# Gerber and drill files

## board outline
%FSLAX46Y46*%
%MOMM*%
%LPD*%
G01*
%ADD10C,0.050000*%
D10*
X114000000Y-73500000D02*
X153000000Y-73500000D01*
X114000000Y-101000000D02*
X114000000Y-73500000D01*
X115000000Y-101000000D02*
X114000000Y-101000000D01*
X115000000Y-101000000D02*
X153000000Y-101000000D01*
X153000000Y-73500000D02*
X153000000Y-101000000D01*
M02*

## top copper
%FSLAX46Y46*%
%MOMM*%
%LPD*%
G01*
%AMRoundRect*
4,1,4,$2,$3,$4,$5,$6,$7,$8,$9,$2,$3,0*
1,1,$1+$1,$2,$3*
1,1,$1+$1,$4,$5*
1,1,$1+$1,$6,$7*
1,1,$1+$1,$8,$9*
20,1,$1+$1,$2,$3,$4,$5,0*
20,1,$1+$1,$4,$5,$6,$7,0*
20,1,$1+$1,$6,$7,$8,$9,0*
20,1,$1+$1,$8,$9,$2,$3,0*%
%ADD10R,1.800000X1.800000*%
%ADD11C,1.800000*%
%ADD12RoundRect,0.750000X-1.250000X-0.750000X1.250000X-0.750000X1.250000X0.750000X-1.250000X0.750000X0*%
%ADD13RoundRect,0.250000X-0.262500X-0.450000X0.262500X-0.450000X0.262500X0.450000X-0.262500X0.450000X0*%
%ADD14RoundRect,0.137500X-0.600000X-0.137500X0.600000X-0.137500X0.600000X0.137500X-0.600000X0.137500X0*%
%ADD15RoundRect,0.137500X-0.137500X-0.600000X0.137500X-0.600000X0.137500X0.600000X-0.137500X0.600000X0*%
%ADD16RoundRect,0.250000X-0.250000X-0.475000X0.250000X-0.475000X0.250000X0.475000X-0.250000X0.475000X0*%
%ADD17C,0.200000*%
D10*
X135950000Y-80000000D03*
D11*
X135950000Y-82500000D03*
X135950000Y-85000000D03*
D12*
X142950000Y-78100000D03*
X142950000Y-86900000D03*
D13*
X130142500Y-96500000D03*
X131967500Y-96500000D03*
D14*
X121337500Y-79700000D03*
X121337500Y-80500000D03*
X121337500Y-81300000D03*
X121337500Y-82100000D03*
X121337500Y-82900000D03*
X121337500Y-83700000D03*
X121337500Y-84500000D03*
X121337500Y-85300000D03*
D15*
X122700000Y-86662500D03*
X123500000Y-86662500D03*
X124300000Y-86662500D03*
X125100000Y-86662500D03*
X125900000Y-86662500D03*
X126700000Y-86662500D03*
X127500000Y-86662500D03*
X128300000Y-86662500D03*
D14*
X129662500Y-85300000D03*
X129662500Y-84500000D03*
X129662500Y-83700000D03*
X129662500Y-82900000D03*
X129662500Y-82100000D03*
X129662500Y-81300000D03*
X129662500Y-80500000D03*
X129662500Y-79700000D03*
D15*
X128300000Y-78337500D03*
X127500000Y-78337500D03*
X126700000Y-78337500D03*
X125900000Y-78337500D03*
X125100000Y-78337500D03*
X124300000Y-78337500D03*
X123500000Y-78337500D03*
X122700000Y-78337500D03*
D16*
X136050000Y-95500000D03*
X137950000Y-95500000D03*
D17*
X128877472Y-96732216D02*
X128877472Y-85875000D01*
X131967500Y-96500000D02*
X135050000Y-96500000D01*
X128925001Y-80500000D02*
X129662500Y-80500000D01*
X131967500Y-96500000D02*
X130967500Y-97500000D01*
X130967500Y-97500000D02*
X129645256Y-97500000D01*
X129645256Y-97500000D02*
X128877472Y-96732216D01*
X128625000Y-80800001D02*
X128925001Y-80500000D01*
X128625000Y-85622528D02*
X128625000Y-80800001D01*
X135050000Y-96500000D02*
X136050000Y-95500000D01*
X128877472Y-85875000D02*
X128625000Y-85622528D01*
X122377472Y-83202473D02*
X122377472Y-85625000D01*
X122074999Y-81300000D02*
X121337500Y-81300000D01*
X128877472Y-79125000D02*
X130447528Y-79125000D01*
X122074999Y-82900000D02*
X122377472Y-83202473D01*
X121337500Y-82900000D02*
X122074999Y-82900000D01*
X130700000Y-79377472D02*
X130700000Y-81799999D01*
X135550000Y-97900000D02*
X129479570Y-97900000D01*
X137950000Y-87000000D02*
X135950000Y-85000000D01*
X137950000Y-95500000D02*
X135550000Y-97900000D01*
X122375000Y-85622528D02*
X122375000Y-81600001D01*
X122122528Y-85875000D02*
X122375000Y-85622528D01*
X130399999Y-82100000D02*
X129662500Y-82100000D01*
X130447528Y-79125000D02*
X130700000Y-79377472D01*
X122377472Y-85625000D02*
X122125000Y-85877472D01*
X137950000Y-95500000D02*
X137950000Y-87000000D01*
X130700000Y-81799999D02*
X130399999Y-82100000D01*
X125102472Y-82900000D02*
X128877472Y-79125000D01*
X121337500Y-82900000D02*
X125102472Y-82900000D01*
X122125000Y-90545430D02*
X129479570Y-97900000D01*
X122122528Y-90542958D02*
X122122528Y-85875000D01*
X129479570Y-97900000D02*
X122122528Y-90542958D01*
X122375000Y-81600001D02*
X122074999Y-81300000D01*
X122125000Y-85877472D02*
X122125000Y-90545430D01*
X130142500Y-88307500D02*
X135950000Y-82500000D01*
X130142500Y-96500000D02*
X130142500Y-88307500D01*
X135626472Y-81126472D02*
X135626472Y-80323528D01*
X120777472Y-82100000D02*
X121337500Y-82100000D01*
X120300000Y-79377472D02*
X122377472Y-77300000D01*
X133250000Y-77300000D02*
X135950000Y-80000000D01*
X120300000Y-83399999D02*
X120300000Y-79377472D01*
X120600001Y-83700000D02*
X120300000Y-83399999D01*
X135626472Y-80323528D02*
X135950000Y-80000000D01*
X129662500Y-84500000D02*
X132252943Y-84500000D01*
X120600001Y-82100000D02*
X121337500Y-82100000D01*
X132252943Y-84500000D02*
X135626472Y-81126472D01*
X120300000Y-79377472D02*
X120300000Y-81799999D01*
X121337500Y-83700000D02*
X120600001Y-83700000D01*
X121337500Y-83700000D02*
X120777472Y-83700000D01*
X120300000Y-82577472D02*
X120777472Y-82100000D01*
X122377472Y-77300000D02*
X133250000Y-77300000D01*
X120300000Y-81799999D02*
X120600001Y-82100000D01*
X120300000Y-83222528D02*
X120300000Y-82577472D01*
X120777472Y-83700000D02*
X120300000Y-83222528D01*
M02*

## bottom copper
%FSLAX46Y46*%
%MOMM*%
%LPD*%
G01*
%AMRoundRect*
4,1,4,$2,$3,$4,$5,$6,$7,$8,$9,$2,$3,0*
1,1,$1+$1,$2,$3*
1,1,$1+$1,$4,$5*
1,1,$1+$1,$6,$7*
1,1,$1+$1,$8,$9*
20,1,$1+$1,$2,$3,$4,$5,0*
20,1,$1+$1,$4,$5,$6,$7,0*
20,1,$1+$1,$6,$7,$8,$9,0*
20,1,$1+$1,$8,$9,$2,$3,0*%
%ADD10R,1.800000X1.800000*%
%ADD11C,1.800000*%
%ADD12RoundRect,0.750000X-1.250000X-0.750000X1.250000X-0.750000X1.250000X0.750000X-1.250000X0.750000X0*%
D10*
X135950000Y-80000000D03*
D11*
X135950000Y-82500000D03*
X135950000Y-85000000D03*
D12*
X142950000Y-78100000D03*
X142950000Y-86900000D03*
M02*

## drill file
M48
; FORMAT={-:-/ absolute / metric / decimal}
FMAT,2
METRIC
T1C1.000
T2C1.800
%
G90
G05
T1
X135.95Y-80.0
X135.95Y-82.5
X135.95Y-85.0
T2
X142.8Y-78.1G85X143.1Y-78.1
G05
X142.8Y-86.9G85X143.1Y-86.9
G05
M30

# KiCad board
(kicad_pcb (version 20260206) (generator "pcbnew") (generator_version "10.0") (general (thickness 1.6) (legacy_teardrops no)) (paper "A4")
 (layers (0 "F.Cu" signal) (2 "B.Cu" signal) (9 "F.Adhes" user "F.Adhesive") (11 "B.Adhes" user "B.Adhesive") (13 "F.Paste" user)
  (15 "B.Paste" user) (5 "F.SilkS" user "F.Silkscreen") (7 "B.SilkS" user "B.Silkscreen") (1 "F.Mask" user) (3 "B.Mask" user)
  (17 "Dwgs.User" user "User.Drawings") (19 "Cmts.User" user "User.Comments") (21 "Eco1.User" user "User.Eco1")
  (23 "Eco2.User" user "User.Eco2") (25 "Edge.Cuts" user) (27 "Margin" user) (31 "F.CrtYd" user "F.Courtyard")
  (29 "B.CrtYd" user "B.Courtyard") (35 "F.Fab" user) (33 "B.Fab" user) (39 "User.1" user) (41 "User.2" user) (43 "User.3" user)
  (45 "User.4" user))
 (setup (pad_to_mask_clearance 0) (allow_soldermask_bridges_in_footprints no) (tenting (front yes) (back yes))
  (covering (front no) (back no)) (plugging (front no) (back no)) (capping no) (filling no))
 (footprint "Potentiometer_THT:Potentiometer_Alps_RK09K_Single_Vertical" (layer "F.Cu") (at 135.95 80)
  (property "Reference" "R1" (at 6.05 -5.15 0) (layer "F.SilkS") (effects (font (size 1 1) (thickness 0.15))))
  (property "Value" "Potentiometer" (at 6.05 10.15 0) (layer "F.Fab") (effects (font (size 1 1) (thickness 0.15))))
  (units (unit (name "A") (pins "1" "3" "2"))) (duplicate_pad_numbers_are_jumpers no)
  (pad "1" thru_hole rect (at 0 0) (size 1.8 1.8) (drill 1) (layers "*.Cu" "*.Mask") (remove_unused_layers no) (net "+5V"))
  (pad "2" thru_hole circle (at 0 2.5) (size 1.8 1.8) (drill 1) (layers "*.Cu" "*.Mask") (remove_unused_layers no) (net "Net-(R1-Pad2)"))
  (pad "3" thru_hole circle (at 0 5) (size 1.8 1.8) (drill 1) (layers "*.Cu" "*.Mask") (remove_unused_layers no) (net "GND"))
  (pad "MP" thru_hole roundrect (at 7 -1.9) (size 4 3) (drill oval 2.1 1.8) (layers "*.Cu" "*.Mask") (remove_unused_layers no)
   (roundrect_rratio 0.25))
  (pad "MP" thru_hole roundrect (at 7 6.9) (size 4 3) (drill oval 2.1 1.8) (layers "*.Cu" "*.Mask") (remove_unused_layers no)
   (roundrect_rratio 0.25)))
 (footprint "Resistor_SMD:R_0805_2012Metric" (layer "F.Cu") (at 131.055 96.5)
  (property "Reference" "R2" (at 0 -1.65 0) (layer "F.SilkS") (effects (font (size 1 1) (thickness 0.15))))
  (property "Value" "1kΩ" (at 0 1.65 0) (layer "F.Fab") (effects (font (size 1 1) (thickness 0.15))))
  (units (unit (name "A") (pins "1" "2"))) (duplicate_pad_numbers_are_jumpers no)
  (pad "1" smd roundrect (at -0.9125 0) (size 1.025 1.4) (layers "F.Cu" "F.Mask" "F.Paste") (roundrect_rratio 0.243902)
   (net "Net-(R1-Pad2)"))
  (pad "2" smd roundrect (at 0.9125 0) (size 1.025 1.4) (layers "F.Cu" "F.Mask" "F.Paste") (roundrect_rratio 0.243902) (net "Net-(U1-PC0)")))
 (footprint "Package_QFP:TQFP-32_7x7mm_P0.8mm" (layer "F.Cu") (at 125.5 82.5)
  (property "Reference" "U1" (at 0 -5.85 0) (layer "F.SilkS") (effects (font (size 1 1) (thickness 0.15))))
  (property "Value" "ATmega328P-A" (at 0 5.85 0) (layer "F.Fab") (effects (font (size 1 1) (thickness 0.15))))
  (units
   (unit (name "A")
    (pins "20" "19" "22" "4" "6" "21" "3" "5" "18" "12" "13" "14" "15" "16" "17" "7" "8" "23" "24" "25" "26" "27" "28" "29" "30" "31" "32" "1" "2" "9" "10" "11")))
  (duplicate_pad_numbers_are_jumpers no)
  (pad "1" smd roundrect (at -4.1625 -2.8) (size 1.475 0.55) (layers "F.Cu" "F.Mask" "F.Paste") (roundrect_rratio 0.25)
   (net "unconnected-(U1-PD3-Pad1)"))
  (pad "2" smd roundrect (at -4.1625 -2) (size 1.475 0.55) (layers "F.Cu" "F.Mask" "F.Paste") (roundrect_rratio 0.25)
   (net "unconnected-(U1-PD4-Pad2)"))
  (pad "3" smd roundrect (at -4.1625 -1.2) (size 1.475 0.55) (layers "F.Cu" "F.Mask" "F.Paste") (roundrect_rratio 0.25) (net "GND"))
  (pad "4" smd roundrect (at -4.1625 -0.4) (size 1.475 0.55) (layers "F.Cu" "F.Mask" "F.Paste") (roundrect_rratio 0.25) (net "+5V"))
  (pad "5" smd roundrect (at -4.1625 0.4) (size 1.475 0.55) (layers "F.Cu" "F.Mask" "F.Paste") (roundrect_rratio 0.25) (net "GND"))
  (pad "6" smd roundrect (at -4.1625 1.2) (size 1.475 0.55) (layers "F.Cu" "F.Mask" "F.Paste") (roundrect_rratio 0.25) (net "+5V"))
  (pad "7" smd roundrect (at -4.1625 2) (size 1.475 0.55) (layers "F.Cu" "F.Mask" "F.Paste") (roundrect_rratio 0.25)
   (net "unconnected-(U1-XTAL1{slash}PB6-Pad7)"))
  (pad "8" smd roundrect (at -4.1625 2.8) (size 1.475 0.55) (layers "F.Cu" "F.Mask" "F.Paste") (roundrect_rratio 0.25)
   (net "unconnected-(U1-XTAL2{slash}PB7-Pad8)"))
  (pad "9" smd roundrect (at -2.8 4.1625) (size 0.55 1.475) (layers "F.Cu" "F.Mask" "F.Paste") (roundrect_rratio 0.25)
   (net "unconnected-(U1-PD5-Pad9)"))
  (pad "10" smd roundrect (at -2 4.1625) (size 0.55 1.475) (layers "F.Cu" "F.Mask" "F.Paste") (roundrect_rratio 0.25)
   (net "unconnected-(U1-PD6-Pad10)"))
  (pad "11" smd roundrect (at -1.2 4.1625) (size 0.55 1.475) (layers "F.Cu" "F.Mask" "F.Paste") (roundrect_rratio 0.25)
   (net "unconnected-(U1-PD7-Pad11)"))
  (pad "12" smd roundrect (at -0.4 4.1625) (size 0.55 1.475) (layers "F.Cu" "F.Mask" "F.Paste") (roundrect_rratio 0.25)
   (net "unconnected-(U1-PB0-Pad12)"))
  (pad "13" smd roundrect (at 0.4 4.1625) (size 0.55 1.475) (layers "F.Cu" "F.Mask" "F.Paste") (roundrect_rratio 0.25)
   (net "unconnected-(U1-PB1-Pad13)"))
  (pad "14" smd roundrect (at 1.2 4.1625) (size 0.55 1.475) (layers "F.Cu" "F.Mask" "F.Paste") (roundrect_rratio 0.25)
   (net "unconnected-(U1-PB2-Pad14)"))
  (pad "15" smd roundrect (at 2 4.1625) (size 0.55 1.475) (layers "F.Cu" "F.Mask" "F.Paste") (roundrect_rratio 0.25)
   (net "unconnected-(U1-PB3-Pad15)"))
  (pad "16" smd roundrect (at 2.8 4.1625) (size 0.55 1.475) (layers "F.Cu" "F.Mask" "F.Paste") (roundrect_rratio 0.25)
   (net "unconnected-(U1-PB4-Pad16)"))
  (pad "17" smd roundrect (at 4.1625 2.8) (size 1.475 0.55) (layers "F.Cu" "F.Mask" "F.Paste") (roundrect_rratio 0.25)
   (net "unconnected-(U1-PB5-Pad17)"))
  (pad "18" smd roundrect (at 4.1625 2) (size 1.475 0.55) (layers "F.Cu" "F.Mask" "F.Paste") (roundrect_rratio 0.25) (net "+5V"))
  (pad "19" smd roundrect (at 4.1625 1.2) (size 1.475 0.55) (layers "F.Cu" "F.Mask" "F.Paste") (roundrect_rratio 0.25)
   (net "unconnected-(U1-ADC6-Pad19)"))
  (pad "20" smd roundrect (at 4.1625 0.4) (size 1.475 0.55) (layers "F.Cu" "F.Mask" "F.Paste") (roundrect_rratio 0.25)
   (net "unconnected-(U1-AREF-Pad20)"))
  (pad "21" smd roundrect (at 4.1625 -0.4) (size 1.475 0.55) (layers "F.Cu" "F.Mask" "F.Paste") (roundrect_rratio 0.25) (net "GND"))
  (pad "22" smd roundrect (at 4.1625 -1.2) (size 1.475 0.55) (layers "F.Cu" "F.Mask" "F.Paste") (roundrect_rratio 0.25)
   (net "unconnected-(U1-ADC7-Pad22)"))
  (pad "23" smd roundrect (at 4.1625 -2) (size 1.475 0.55) (layers "F.Cu" "F.Mask" "F.Paste") (roundrect_rratio 0.25) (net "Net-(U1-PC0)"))
  (pad "24" smd roundrect (at 4.1625 -2.8) (size 1.475 0.55) (layers "F.Cu" "F.Mask" "F.Paste") (roundrect_rratio 0.25)
   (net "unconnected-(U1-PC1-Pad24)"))
  (pad "25" smd roundrect (at 2.8 -4.1625) (size 0.55 1.475) (layers "F.Cu" "F.Mask" "F.Paste") (roundrect_rratio 0.25)
   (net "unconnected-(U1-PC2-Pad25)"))
  (pad "26" smd roundrect (at 2 -4.1625) (size 0.55 1.475) (layers "F.Cu" "F.Mask" "F.Paste") (roundrect_rratio 0.25)
   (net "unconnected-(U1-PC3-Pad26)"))
  (pad "27" smd roundrect (at 1.2 -4.1625) (size 0.55 1.475) (layers "F.Cu" "F.Mask" "F.Paste") (roundrect_rratio 0.25)
   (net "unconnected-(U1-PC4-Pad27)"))
  (pad "28" smd roundrect (at 0.4 -4.1625) (size 0.55 1.475) (layers "F.Cu" "F.Mask" "F.Paste") (roundrect_rratio 0.25)
   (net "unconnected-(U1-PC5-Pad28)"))
  (pad "29" smd roundrect (at -0.4 -4.1625) (size 0.55 1.475) (layers "F.Cu" "F.Mask" "F.Paste") (roundrect_rratio 0.25)
   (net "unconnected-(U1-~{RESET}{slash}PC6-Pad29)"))
  (pad "30" smd roundrect (at -1.2 -4.1625) (size 0.55 1.475) (layers "F.Cu" "F.Mask" "F.Paste") (roundrect_rratio 0.25)
   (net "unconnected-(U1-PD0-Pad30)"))
  (pad "31" smd roundrect (at -2 -4.1625) (size 0.55 1.475) (layers "F.Cu" "F.Mask" "F.Paste") (roundrect_rratio 0.25)
   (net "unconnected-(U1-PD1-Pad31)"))
  (pad "32" smd roundrect (at -2.8 -4.1625) (size 0.55 1.475) (layers "F.Cu" "F.Mask" "F.Paste") (roundrect_rratio 0.25)
   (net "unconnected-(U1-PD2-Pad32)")))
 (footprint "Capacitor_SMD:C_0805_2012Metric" (layer "F.Cu") (at 137 95.5)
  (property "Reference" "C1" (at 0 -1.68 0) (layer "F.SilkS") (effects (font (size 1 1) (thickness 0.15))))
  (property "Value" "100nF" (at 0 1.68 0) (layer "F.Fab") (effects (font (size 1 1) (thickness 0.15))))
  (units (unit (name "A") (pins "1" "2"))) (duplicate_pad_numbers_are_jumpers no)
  (pad "1" smd roundrect (at -0.95 0) (size 1 1.45) (layers "F.Cu" "F.Mask" "F.Paste") (roundrect_rratio 0.25) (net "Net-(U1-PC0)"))
  (pad "2" smd roundrect (at 0.95 0) (size 1 1.45) (layers "F.Cu" "F.Mask" "F.Paste") (roundrect_rratio 0.25) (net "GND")))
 (gr_line (start 114 73.5) (end 153 73.5) (stroke (width 0.05) (type default)) (layer "Edge.Cuts"))
 (gr_line (start 114 101) (end 114 73.5) (stroke (width 0.05) (type default)) (layer "Edge.Cuts"))
 (gr_line (start 115 101) (end 114 101) (stroke (width 0.05) (type default)) (layer "Edge.Cuts"))
 (gr_line (start 115 101) (end 153 101) (stroke (width 0.05) (type default)) (layer "Edge.Cuts"))
 (gr_line (start 153 73.5) (end 153 101) (stroke (width 0.05) (type default)) (layer "Edge.Cuts"))
 (segment (start 128.877472 96.732216) (end 128.877472 85.875) (width 0.2) (layer "F.Cu") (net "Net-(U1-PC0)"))
 (segment (start 131.9675 96.5) (end 135.05 96.5) (width 0.2) (layer "F.Cu") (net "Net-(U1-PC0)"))
 (segment (start 128.925001 80.5) (end 129.6625 80.5) (width 0.2) (layer "F.Cu") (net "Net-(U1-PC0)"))
 (segment (start 131.9675 96.5) (end 130.9675 97.5) (width 0.2) (layer "F.Cu") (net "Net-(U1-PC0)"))
 (segment (start 130.9675 97.5) (end 129.645256 97.5) (width 0.2) (layer "F.Cu") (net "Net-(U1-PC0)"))
 (segment (start 129.645256 97.5) (end 128.877472 96.732216) (width 0.2) (layer "F.Cu") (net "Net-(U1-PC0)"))
 (segment (start 128.625 80.800001) (end 128.925001 80.5) (width 0.2) (layer "F.Cu") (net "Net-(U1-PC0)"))
 (segment (start 128.625 85.622528) (end 128.625 80.800001) (width 0.2) (layer "F.Cu") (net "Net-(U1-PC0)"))
 (segment (start 135.05 96.5) (end 136.05 95.5) (width 0.2) (layer "F.Cu") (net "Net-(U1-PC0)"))
 (segment (start 128.877472 85.875) (end 128.625 85.622528) (width 0.2) (layer "F.Cu") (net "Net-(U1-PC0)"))
 (segment (start 122.377472 83.202473) (end 122.377472 85.625) (width 0.2) (layer "F.Cu") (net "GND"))
 (segment (start 122.074999 81.3) (end 121.3375 81.3) (width 0.2) (layer "F.Cu") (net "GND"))
 (segment (start 128.877472 79.125) (end 130.447528 79.125) (width 0.2) (layer "F.Cu") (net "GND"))
 (segment (start 122.074999 82.9) (end 122.377472 83.202473) (width 0.2) (layer "F.Cu") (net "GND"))
 (segment (start 121.3375 82.9) (end 122.074999 82.9) (width 0.2) (layer "F.Cu") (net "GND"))
 (segment (start 130.7 79.377472) (end 130.7 81.799999) (width 0.2) (layer "F.Cu") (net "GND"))
 (segment (start 135.55 97.9) (end 129.47957 97.9) (width 0.2) (layer "F.Cu") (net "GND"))
 (segment (start 137.95 87) (end 135.95 85) (width 0.2) (layer "F.Cu") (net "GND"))
 (segment (start 137.95 95.5) (end 135.55 97.9) (width 0.2) (layer "F.Cu") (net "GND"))
 (segment (start 122.375 85.622528) (end 122.375 81.600001) (width 0.2) (layer "F.Cu") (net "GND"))
 (segment (start 122.122528 85.875) (end 122.375 85.622528) (width 0.2) (layer "F.Cu") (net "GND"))
 (segment (start 130.399999 82.1) (end 129.6625 82.1) (width 0.2) (layer "F.Cu") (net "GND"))
 (segment (start 130.447528 79.125) (end 130.7 79.377472) (width 0.2) (layer "F.Cu") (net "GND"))
 (segment (start 122.377472 85.625) (end 122.125 85.877472) (width 0.2) (layer "F.Cu") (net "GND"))
 (segment (start 137.95 95.5) (end 137.95 87) (width 0.2) (layer "F.Cu") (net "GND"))
 (segment (start 130.7 81.799999) (end 130.399999 82.1) (width 0.2) (layer "F.Cu") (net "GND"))
 (segment (start 125.102472 82.9) (end 128.877472 79.125) (width 0.2) (layer "F.Cu") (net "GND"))
 (segment (start 121.3375 82.9) (end 125.102472 82.9) (width 0.2) (layer "F.Cu") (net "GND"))
 (segment (start 122.125 90.54543) (end 129.47957 97.9) (width 0.2) (layer "F.Cu") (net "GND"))
 (segment (start 122.122528 90.542958) (end 122.122528 85.875) (width 0.2) (layer "F.Cu") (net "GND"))
 (segment (start 129.47957 97.9) (end 122.122528 90.542958) (width 0.2) (layer "F.Cu") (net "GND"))
 (segment (start 122.375 81.600001) (end 122.074999 81.3) (width 0.2) (layer "F.Cu") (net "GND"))
 (segment (start 122.125 85.877472) (end 122.125 90.54543) (width 0.2) (layer "F.Cu") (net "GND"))
 (segment (start 130.1425 88.3075) (end 135.95 82.5) (width 0.2) (layer "F.Cu") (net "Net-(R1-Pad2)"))
 (segment (start 130.1425 96.5) (end 130.1425 88.3075) (width 0.2) (layer "F.Cu") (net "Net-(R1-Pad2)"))
 (segment (start 135.626472 81.126472) (end 135.626472 80.323528) (width 0.2) (layer "F.Cu") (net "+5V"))
 (segment (start 120.777472 82.1) (end 121.3375 82.1) (width 0.2) (layer "F.Cu") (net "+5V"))
 (segment (start 120.3 79.377472) (end 122.377472 77.3) (width 0.2) (layer "F.Cu") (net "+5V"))
 (segment (start 133.25 77.3) (end 135.95 80) (width 0.2) (layer "F.Cu") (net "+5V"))
 (segment (start 120.3 83.399999) (end 120.3 79.377472) (width 0.2) (layer "F.Cu") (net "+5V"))
 (segment (start 120.600001 83.7) (end 120.3 83.399999) (width 0.2) (layer "F.Cu") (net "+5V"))
 (segment (start 135.626472 80.323528) (end 135.95 80) (width 0.2) (layer "F.Cu") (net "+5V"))
 (segment (start 129.6625 84.5) (end 132.252943 84.5) (width 0.2) (layer "F.Cu") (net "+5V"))
 (segment (start 120.600001 82.1) (end 121.3375 82.1) (width 0.2) (layer "F.Cu") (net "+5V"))
 (segment (start 132.252943 84.5) (end 135.626472 81.126472) (width 0.2) (layer "F.Cu") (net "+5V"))
 (segment (start 120.3 79.377472) (end 120.3 81.799999) (width 0.2) (layer "F.Cu") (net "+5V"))
 (segment (start 121.3375 83.7) (end 120.600001 83.7) (width 0.2) (layer "F.Cu") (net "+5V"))
 (segment (start 121.3375 83.7) (end 120.777472 83.7) (width 0.2) (layer "F.Cu") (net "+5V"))
 (segment (start 120.3 82.577472) (end 120.777472 82.1) (width 0.2) (layer "F.Cu") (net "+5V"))
 (segment (start 122.377472 77.3) (end 133.25 77.3) (width 0.2) (layer "F.Cu") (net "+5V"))
 (segment (start 120.3 81.799999) (end 120.600001 82.1) (width 0.2) (layer "F.Cu") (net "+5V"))
 (segment (start 120.3 83.222528) (end 120.3 82.577472) (width 0.2) (layer "F.Cu") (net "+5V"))
 (segment (start 120.777472 83.7) (end 120.3 83.222528) (width 0.2) (layer "F.Cu") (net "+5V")))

